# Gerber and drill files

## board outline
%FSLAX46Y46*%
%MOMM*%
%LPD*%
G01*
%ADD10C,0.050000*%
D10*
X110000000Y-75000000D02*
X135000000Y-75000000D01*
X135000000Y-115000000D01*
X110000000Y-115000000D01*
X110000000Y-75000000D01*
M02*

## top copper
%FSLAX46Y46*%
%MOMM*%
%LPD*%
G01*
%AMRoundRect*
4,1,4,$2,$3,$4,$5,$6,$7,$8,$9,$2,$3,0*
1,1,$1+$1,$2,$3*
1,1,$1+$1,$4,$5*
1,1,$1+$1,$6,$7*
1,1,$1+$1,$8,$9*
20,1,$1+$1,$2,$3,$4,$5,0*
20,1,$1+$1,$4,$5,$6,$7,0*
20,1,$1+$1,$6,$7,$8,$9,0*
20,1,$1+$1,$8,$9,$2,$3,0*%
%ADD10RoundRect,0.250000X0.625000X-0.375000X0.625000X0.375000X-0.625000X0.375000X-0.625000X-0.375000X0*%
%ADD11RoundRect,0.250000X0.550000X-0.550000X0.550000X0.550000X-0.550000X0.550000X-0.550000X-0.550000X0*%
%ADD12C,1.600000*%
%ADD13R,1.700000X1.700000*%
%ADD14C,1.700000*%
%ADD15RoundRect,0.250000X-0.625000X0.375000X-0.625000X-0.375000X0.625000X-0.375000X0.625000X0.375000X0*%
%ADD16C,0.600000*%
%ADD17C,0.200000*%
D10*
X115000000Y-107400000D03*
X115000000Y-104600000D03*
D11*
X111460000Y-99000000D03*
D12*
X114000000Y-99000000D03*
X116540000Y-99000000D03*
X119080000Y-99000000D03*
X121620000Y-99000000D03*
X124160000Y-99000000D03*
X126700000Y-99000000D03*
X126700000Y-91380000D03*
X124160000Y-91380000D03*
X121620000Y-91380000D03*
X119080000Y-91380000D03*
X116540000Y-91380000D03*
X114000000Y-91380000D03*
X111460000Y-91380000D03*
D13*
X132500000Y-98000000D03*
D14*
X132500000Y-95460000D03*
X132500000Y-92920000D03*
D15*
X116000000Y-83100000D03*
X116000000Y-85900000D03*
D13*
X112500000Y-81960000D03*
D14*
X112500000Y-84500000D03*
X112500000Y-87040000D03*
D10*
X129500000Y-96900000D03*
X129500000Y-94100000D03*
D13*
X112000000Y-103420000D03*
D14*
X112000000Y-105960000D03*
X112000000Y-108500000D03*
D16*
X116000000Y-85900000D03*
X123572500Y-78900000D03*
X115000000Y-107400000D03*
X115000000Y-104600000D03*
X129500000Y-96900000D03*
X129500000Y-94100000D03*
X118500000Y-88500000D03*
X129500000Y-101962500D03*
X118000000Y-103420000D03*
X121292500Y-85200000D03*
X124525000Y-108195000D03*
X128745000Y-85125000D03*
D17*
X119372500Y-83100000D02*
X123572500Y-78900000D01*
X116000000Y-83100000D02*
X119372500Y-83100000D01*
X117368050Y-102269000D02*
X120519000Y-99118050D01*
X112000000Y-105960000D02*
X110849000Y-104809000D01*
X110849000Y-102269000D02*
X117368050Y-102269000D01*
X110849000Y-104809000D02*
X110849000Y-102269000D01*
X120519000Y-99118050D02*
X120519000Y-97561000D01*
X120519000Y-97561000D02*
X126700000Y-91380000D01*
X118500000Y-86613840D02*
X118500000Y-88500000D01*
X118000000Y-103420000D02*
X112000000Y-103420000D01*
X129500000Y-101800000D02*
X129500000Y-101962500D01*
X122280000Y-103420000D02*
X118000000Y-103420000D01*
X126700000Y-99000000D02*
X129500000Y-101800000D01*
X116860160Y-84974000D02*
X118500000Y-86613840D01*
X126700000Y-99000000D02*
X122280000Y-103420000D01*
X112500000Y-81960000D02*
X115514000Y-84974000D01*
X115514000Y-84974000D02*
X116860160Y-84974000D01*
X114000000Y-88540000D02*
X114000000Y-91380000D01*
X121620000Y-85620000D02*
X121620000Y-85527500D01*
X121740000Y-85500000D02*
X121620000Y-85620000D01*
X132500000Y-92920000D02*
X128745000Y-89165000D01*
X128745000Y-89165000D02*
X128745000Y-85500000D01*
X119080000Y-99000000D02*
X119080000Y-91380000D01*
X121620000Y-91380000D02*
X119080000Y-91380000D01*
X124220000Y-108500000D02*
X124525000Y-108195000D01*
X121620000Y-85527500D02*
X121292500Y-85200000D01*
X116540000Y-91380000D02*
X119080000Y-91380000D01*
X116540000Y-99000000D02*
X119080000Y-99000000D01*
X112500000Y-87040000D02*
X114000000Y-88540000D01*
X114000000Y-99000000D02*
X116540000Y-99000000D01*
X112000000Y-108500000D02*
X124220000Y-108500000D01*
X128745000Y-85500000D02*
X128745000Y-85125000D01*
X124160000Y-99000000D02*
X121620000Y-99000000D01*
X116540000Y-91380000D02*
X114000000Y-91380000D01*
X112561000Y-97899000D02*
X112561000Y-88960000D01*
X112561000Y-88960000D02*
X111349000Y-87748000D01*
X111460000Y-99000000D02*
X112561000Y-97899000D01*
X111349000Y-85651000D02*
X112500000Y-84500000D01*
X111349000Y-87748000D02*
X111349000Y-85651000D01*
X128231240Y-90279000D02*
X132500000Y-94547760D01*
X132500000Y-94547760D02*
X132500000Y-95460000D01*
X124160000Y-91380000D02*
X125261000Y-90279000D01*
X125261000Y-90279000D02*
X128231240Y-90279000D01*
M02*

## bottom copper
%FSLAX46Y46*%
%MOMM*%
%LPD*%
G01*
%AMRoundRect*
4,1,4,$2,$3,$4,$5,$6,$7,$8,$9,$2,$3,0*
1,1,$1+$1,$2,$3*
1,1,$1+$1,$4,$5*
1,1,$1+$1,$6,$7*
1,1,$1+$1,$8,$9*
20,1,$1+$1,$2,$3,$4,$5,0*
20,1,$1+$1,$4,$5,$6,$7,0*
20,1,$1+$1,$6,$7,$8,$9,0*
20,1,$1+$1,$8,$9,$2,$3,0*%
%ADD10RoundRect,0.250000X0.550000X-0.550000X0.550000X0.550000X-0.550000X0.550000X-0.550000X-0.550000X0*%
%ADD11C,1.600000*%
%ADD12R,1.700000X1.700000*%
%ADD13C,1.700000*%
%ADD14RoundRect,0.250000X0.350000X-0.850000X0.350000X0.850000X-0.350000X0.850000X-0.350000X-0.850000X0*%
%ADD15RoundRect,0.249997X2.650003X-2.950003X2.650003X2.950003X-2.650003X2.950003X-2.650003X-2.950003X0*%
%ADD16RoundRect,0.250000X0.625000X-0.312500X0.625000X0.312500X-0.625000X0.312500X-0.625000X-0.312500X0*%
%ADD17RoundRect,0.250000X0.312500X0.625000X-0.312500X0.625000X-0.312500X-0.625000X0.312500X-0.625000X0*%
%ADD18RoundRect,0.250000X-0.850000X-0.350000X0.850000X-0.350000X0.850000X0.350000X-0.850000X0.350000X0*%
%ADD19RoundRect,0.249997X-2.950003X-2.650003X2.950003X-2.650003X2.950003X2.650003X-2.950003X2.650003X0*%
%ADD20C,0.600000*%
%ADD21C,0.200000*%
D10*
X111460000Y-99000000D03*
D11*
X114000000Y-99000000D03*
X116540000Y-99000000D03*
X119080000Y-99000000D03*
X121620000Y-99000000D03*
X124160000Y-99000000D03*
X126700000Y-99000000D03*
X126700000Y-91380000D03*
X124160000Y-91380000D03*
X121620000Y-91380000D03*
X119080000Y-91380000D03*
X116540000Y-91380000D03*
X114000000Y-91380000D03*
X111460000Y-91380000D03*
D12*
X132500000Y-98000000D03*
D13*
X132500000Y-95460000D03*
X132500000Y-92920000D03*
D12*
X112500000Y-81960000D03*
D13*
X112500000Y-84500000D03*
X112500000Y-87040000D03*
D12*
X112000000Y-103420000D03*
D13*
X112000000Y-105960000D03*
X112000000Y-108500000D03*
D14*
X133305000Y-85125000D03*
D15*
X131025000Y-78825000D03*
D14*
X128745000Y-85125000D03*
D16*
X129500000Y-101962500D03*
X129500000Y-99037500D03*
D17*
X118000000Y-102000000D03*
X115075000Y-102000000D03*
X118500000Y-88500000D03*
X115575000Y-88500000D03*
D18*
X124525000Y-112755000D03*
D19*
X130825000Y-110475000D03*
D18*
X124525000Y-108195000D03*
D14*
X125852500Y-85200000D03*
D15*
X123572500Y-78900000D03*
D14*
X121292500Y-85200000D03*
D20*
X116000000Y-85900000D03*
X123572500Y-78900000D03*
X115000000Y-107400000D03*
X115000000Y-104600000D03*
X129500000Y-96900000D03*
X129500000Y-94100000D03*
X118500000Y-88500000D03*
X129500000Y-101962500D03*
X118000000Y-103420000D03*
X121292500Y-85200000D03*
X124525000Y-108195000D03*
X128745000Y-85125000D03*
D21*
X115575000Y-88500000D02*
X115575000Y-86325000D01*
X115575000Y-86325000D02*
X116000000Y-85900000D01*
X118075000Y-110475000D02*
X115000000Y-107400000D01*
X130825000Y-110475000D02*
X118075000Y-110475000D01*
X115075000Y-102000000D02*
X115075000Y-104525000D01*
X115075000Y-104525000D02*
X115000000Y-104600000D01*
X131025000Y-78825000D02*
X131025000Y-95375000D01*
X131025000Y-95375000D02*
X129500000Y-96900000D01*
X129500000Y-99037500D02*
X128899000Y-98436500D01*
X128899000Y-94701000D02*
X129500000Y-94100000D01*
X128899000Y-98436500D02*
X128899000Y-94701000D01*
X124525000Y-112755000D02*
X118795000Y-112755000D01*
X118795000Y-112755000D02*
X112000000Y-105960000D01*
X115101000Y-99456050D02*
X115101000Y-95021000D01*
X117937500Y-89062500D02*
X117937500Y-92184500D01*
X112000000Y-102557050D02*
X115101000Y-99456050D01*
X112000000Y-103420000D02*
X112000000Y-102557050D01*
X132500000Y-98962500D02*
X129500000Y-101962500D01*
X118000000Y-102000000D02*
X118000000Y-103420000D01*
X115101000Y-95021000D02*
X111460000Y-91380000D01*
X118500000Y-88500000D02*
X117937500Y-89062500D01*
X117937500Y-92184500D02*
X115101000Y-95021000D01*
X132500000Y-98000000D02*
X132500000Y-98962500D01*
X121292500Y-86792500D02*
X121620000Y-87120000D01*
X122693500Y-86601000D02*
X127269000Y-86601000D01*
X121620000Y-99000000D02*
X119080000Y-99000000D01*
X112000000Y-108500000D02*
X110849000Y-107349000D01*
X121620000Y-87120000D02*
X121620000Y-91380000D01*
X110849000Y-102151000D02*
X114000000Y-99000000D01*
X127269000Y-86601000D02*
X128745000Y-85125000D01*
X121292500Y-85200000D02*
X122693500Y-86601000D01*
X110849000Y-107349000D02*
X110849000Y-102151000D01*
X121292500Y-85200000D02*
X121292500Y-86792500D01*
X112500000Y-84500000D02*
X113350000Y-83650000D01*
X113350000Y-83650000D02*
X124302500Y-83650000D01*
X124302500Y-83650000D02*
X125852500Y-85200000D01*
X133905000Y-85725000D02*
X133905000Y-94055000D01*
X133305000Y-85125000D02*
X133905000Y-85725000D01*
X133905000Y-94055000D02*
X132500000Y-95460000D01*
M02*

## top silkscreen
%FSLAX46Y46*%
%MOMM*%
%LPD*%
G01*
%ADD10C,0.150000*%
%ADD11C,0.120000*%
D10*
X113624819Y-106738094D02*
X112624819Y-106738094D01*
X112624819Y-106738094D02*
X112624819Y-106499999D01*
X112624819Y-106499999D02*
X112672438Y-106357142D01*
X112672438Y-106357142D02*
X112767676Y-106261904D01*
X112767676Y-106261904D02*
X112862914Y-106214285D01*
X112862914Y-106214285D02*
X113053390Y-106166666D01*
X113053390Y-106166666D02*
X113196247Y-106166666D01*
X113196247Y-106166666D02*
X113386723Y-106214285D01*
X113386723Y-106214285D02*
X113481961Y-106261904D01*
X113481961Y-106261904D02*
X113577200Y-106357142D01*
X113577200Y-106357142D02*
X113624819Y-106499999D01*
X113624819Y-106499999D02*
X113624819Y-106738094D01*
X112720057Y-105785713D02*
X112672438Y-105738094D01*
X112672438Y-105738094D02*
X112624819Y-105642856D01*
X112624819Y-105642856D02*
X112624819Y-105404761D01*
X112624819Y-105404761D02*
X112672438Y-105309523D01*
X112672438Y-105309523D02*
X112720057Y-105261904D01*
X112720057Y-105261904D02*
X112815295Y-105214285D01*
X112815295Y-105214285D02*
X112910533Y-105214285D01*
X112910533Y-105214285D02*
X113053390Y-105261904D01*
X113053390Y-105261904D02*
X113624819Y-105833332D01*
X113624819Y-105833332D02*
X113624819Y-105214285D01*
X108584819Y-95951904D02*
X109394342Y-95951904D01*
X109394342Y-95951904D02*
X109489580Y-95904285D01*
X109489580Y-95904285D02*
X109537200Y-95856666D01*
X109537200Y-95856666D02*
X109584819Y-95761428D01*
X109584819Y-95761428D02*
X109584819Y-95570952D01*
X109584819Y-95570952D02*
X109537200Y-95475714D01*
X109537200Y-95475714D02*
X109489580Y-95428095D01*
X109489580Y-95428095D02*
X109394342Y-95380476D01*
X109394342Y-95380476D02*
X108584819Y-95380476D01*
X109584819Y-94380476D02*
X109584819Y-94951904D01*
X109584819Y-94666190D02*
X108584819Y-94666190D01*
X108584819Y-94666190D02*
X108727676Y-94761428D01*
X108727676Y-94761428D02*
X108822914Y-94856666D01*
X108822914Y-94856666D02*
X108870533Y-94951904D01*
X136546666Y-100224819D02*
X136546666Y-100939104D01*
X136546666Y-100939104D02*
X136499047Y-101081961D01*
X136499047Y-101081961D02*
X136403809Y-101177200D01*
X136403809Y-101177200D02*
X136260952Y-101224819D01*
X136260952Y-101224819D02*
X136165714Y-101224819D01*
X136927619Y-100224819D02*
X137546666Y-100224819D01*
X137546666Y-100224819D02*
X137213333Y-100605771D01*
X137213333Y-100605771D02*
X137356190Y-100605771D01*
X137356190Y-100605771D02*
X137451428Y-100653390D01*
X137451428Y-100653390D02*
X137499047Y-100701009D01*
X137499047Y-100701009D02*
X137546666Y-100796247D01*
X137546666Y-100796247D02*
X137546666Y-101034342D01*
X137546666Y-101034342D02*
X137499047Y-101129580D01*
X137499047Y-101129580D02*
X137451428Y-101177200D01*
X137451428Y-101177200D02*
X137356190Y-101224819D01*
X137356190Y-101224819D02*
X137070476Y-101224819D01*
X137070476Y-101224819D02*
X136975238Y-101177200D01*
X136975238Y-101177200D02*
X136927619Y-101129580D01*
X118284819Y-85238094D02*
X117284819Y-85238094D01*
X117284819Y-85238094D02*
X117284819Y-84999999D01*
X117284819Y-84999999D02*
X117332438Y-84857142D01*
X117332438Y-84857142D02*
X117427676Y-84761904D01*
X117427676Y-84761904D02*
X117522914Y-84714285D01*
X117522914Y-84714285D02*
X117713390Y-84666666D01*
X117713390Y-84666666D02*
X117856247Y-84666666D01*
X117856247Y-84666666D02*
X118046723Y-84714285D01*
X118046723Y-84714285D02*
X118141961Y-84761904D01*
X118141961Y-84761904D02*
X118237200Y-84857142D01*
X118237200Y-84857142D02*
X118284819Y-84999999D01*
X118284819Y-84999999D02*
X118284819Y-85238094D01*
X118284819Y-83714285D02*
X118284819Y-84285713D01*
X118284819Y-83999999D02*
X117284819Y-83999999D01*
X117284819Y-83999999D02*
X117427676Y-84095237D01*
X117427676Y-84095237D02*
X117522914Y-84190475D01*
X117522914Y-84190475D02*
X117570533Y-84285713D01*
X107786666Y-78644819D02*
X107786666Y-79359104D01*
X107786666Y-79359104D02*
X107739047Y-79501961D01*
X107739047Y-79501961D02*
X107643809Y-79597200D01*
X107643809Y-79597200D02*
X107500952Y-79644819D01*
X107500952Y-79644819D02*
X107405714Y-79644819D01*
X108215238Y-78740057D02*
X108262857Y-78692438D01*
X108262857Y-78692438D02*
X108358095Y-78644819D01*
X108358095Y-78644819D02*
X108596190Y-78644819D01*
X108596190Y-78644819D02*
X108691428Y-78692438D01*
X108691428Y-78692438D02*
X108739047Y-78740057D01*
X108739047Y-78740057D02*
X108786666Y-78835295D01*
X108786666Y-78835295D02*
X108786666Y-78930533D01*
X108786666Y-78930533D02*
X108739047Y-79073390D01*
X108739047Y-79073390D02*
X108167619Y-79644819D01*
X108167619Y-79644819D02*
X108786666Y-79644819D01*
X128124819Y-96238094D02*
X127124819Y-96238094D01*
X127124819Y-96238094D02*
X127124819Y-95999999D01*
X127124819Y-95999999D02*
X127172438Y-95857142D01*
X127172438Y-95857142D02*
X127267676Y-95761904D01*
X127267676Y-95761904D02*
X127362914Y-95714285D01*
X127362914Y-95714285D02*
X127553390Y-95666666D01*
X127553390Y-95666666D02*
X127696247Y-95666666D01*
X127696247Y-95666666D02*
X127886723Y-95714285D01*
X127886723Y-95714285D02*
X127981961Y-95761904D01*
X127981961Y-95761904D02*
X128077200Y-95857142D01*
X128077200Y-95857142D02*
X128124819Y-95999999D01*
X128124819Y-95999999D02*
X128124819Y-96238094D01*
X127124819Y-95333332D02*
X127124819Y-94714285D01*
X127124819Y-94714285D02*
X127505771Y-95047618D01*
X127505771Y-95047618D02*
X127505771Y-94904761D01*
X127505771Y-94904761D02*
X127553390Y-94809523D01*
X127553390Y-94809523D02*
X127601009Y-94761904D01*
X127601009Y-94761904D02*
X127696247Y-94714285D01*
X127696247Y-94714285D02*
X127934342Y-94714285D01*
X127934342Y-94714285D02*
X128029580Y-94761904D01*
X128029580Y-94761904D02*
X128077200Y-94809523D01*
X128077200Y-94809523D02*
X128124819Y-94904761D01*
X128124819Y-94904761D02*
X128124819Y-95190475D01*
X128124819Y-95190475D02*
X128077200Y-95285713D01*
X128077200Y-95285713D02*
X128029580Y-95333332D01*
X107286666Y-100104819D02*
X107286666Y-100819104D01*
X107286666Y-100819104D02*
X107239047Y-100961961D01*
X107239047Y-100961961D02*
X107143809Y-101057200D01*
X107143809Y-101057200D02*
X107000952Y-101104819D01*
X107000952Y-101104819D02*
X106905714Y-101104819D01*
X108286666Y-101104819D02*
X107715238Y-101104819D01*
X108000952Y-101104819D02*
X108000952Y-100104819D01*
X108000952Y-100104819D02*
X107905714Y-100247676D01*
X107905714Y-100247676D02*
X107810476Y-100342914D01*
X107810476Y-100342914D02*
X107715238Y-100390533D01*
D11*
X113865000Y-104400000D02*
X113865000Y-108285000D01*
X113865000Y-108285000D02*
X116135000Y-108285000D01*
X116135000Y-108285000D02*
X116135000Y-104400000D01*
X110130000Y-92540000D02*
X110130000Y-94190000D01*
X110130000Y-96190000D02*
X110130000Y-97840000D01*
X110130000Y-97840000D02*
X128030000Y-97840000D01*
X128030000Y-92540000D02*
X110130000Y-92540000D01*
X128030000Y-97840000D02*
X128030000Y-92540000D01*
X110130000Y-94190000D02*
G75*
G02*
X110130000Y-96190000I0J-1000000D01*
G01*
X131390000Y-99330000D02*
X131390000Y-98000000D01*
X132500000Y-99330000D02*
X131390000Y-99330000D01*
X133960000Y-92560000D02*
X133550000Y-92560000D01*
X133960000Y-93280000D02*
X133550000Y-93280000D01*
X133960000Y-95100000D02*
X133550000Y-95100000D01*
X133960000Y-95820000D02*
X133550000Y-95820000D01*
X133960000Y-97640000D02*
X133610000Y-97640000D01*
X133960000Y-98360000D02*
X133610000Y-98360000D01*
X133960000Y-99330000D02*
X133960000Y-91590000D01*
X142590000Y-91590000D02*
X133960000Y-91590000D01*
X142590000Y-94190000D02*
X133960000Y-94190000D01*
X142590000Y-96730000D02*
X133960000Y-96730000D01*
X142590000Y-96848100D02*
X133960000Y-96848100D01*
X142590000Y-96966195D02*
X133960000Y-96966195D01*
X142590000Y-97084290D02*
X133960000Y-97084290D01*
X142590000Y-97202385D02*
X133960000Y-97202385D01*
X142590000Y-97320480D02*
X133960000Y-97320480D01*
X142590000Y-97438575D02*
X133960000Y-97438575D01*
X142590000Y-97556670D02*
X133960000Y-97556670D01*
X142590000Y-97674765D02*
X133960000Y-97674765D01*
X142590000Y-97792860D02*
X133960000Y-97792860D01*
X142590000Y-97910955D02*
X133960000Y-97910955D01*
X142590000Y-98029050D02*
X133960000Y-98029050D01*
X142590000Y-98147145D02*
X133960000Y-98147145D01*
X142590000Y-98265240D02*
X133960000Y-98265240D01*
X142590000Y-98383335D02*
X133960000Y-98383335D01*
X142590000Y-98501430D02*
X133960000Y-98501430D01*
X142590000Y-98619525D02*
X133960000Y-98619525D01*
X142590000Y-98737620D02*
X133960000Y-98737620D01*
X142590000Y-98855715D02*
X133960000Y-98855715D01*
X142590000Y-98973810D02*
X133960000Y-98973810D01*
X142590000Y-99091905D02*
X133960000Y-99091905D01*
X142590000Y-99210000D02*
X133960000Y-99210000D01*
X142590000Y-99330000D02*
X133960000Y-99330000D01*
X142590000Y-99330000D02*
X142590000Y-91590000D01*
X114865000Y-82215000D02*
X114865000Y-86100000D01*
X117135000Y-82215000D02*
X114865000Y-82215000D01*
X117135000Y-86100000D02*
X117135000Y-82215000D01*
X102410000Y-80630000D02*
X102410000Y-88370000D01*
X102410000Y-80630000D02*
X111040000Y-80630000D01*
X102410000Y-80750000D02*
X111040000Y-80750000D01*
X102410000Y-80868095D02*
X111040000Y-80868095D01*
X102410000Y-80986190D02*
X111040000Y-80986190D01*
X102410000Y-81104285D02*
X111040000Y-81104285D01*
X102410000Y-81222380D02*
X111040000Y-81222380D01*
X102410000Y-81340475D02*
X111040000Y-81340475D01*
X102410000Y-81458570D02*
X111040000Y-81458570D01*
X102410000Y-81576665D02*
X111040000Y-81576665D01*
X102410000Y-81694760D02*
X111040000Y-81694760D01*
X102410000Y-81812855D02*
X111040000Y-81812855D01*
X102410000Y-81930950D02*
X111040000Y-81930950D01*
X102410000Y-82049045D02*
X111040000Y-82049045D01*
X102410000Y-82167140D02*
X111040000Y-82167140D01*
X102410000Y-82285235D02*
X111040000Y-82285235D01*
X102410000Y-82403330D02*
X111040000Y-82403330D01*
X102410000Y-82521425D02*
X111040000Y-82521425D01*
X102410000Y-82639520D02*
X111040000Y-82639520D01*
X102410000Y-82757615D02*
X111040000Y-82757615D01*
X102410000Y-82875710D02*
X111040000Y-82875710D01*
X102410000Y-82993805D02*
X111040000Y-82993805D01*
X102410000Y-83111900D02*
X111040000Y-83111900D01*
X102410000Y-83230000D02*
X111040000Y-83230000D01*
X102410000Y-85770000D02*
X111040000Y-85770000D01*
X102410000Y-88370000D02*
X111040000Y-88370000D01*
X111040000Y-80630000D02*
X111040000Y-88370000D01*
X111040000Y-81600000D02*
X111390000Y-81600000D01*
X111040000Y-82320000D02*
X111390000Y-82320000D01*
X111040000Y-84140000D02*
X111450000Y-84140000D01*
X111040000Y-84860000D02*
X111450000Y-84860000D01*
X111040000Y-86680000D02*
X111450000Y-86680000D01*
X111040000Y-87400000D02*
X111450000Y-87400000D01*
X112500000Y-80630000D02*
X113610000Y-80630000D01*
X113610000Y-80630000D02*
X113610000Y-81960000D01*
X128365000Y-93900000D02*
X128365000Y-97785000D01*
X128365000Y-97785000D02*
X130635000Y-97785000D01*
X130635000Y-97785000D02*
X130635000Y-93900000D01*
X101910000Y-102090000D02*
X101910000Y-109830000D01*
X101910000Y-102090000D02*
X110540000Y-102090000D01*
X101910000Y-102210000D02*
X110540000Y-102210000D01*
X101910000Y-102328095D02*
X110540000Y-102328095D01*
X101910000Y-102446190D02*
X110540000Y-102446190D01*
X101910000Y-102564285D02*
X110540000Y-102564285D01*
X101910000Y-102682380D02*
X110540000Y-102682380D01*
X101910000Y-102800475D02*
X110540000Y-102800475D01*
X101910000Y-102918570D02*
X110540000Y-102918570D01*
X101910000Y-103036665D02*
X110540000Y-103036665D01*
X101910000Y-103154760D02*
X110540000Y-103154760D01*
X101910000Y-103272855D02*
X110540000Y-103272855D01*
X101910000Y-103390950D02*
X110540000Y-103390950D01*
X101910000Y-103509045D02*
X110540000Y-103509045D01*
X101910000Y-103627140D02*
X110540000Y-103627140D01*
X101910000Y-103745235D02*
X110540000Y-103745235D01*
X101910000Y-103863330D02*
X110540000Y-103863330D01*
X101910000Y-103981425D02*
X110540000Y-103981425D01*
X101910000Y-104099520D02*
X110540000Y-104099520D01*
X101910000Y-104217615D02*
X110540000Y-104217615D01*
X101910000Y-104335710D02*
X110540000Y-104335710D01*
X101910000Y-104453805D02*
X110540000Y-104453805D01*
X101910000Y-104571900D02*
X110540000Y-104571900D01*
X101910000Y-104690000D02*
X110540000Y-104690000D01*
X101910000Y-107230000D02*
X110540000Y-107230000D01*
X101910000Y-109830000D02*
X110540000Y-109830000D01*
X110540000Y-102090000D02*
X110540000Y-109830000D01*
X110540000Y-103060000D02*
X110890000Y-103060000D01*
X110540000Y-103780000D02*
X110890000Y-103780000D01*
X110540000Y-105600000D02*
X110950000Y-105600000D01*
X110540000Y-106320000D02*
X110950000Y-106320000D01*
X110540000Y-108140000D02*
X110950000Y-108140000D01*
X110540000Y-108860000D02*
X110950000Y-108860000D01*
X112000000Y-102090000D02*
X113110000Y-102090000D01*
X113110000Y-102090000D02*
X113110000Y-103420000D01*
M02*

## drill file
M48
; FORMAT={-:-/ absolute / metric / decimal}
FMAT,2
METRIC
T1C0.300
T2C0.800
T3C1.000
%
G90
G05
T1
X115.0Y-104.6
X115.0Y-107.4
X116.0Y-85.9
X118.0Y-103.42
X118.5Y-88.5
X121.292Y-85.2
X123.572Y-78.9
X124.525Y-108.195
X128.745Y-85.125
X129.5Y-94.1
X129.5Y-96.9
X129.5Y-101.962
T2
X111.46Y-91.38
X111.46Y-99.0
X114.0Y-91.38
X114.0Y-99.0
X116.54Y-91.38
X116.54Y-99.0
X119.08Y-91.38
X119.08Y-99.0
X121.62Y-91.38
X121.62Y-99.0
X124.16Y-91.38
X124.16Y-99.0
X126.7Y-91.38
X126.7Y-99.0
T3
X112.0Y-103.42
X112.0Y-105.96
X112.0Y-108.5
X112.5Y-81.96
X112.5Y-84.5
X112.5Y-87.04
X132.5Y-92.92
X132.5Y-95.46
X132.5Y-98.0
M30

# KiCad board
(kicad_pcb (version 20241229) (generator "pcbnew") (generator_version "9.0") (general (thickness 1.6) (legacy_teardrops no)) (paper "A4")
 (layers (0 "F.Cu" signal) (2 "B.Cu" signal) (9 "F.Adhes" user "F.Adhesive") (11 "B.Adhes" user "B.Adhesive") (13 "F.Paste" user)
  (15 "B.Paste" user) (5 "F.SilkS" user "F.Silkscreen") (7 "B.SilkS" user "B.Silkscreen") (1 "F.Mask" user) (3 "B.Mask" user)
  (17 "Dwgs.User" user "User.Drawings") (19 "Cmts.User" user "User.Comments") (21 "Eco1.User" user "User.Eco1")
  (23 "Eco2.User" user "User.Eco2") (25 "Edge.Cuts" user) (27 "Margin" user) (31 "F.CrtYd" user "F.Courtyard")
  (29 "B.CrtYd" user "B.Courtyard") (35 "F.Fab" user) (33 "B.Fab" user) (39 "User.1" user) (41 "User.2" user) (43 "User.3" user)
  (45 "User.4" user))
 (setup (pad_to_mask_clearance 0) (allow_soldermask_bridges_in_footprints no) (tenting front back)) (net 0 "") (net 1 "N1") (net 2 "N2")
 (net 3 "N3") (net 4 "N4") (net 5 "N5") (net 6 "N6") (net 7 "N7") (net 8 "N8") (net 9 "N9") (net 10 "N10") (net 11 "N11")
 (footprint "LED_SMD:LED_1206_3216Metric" (layer "F.Cu") (at 115 106 90)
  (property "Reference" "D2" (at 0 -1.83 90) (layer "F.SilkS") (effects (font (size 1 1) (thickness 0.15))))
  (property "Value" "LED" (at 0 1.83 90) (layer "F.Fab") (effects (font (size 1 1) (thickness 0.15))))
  (fp_line (start 1.6 -1.135) (end -2.285 -1.135) (stroke (width 0.12) (type solid)) (layer "F.SilkS"))
  (fp_line (start -2.285 -1.135) (end -2.285 1.135) (stroke (width 0.12) (type solid)) (layer "F.SilkS"))
  (fp_line (start -2.285 1.135) (end 1.6 1.135) (stroke (width 0.12) (type solid)) (layer "F.SilkS"))
  (pad "1" smd roundrect (at -1.4 0 90) (size 1.25 1.75) (layers "F.Cu" "F.Mask" "F.Paste") (roundrect_rratio 0.2) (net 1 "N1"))
  (pad "2" smd roundrect (at 1.4 0 90) (size 1.25 1.75) (layers "F.Cu" "F.Mask" "F.Paste") (roundrect_rratio 0.2) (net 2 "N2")))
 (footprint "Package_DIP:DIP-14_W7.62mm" (layer "F.Cu") (at 111.46 99 90)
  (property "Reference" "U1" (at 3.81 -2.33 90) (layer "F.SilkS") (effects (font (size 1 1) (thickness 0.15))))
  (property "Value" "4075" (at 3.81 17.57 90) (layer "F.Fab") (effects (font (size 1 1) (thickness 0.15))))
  (fp_line (start 6.46 -1.33) (end 4.81 -1.33) (stroke (width 0.12) (type solid)) (layer "F.SilkS"))
  (fp_line (start 2.81 -1.33) (end 1.16 -1.33) (stroke (width 0.12) (type solid)) (layer "F.SilkS"))
  (fp_line (start 1.16 -1.33) (end 1.16 16.57) (stroke (width 0.12) (type solid)) (layer "F.SilkS"))
  (fp_line (start 6.46 16.57) (end 6.46 -1.33) (stroke (width 0.12) (type solid)) (layer "F.SilkS"))
  (fp_line (start 1.16 16.57) (end 6.46 16.57) (stroke (width 0.12) (type solid)) (layer "F.SilkS"))
  (fp_arc (start 4.81 -1.33) (mid 3.81 -0.33) (end 2.81 -1.33) (stroke (width 0.12) (type solid)) (layer "F.SilkS"))
  (pad "1" thru_hole roundrect (at 0 0 90) (size 1.6 1.6) (drill 0.8) (layers "*.Cu" "*.Mask") (remove_unused_layers no)
   (roundrect_rratio 0.15625) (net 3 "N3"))
  (pad "2" thru_hole circle (at 0 2.54 90) (size 1.6 1.6) (drill 0.8) (layers "*.Cu" "*.Mask") (remove_unused_layers no) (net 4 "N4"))
  (pad "3" thru_hole circle (at 0 5.08 90) (size 1.6 1.6) (drill 0.8) (layers "*.Cu" "*.Mask") (remove_unused_layers no) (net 4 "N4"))
  (pad "4" thru_hole circle (at 0 7.62 90) (size 1.6 1.6) (drill 0.8) (layers "*.Cu" "*.Mask") (remove_unused_layers no) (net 4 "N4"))
  (pad "5" thru_hole circle (at 0 10.16 90) (size 1.6 1.6) (drill 0.8) (layers "*.Cu" "*.Mask") (remove_unused_layers no) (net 4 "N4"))
  (pad "6" thru_hole circle (at 0 12.7 90) (size 1.6 1.6) (drill 0.8) (layers "*.Cu" "*.Mask") (remove_unused_layers no) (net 4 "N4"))
  (pad "7" thru_hole circle (at 0 15.24 90) (size 1.6 1.6) (drill 0.8) (layers "*.Cu" "*.Mask") (remove_unused_layers no) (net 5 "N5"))
  (pad "8" thru_hole circle (at 7.62 15.24 90) (size 1.6 1.6) (drill 0.8) (layers "*.Cu" "*.Mask") (remove_unused_layers no) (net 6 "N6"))
  (pad "9" thru_hole circle (at 7.62 12.7 90) (size 1.6 1.6) (drill 0.8) (layers "*.Cu" "*.Mask") (remove_unused_layers no) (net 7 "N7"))
  (pad "10" thru_hole circle (at 7.62 10.16 90) (size 1.6 1.6) (drill 0.8) (layers "*.Cu" "*.Mask") (remove_unused_layers no) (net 4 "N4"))
  (pad "11" thru_hole circle (at 7.62 7.62 90) (size 1.6 1.6) (drill 0.8) (layers "*.Cu" "*.Mask") (remove_unused_layers no) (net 4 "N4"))
  (pad "12" thru_hole circle (at 7.62 5.08 90) (size 1.6 1.6) (drill 0.8) (layers "*.Cu" "*.Mask") (remove_unused_layers no) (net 4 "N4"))
  (pad "13" thru_hole circle (at 7.62 2.54 90) (size 1.6 1.6) (drill 0.8) (layers "*.Cu" "*.Mask") (remove_unused_layers no) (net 4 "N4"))
  (pad "14" thru_hole circle (at 7.62 0 90) (size 1.6 1.6) (drill 0.8) (layers "*.Cu" "*.Mask") (remove_unused_layers no) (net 5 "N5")))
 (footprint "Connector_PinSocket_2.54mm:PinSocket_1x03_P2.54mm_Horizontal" (layer "F.Cu") (at 132.5 98 180)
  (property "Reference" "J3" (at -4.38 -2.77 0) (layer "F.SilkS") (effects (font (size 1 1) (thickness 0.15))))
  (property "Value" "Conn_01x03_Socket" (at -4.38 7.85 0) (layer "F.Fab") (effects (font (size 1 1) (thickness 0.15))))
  (fp_line (start 1.11 -1.33) (end 1.11 0) (stroke (width 0.12) (type solid)) (layer "F.SilkS"))
  (fp_line (start 0 -1.33) (end 1.11 -1.33) (stroke (width 0.12) (type solid)) (layer "F.SilkS"))
  (fp_line (start -1.46 5.44) (end -1.05 5.44) (stroke (width 0.12) (type solid)) (layer "F.SilkS"))
  (fp_line (start -1.46 4.72) (end -1.05 4.72) (stroke (width 0.12) (type solid)) (layer "F.SilkS"))
  (fp_line (start -1.46 2.9) (end -1.05 2.9) (stroke (width 0.12) (type solid)) (layer "F.SilkS"))
  (fp_line (start -1.46 2.18) (end -1.05 2.18) (stroke (width 0.12) (type solid)) (layer "F.SilkS"))
  (fp_line (start -1.46 0.36) (end -1.11 0.36) (stroke (width 0.12) (type solid)) (layer "F.SilkS"))
  (fp_line (start -1.46 -0.36) (end -1.11 -0.36) (stroke (width 0.12) (type solid)) (layer "F.SilkS"))
  (fp_line (start -1.46 -1.33) (end -1.46 6.41) (stroke (width 0.12) (type solid)) (layer "F.SilkS"))
  (fp_line (start -10.09 6.41) (end -1.46 6.41) (stroke (width 0.12) (type solid)) (layer "F.SilkS"))
  (fp_line (start -10.09 3.81) (end -1.46 3.81) (stroke (width 0.12) (type solid)) (layer "F.SilkS"))
  (fp_line (start -10.09 1.27) (end -1.46 1.27) (stroke (width 0.12) (type solid)) (layer "F.SilkS"))
  (fp_line (start -10.09 1.1519) (end -1.46 1.1519) (stroke (width 0.12) (type solid)) (layer "F.SilkS"))
  (fp_line (start -10.09 1.033805) (end -1.46 1.033805) (stroke (width 0.12) (type solid)) (layer "F.SilkS"))
  (fp_line (start -10.09 0.91571) (end -1.46 0.91571) (stroke (width 0.12) (type solid)) (layer "F.SilkS"))
  (fp_line (start -10.09 0.797615) (end -1.46 0.797615) (stroke (width 0.12) (type solid)) (layer "F.SilkS"))
  (fp_line (start -10.09 0.67952) (end -1.46 0.67952) (stroke (width 0.12) (type solid)) (layer "F.SilkS"))
  (fp_line (start -10.09 0.561425) (end -1.46 0.561425) (stroke (width 0.12) (type solid)) (layer "F.SilkS"))
  (fp_line (start -10.09 0.44333) (end -1.46 0.44333) (stroke (width 0.12) (type solid)) (layer "F.SilkS"))
  (fp_line (start -10.09 0.325235) (end -1.46 0.325235) (stroke (width 0.12) (type solid)) (layer "F.SilkS"))
  (fp_line (start -10.09 0.20714) (end -1.46 0.20714) (stroke (width 0.12) (type solid)) (layer "F.SilkS"))
  (fp_line (start -10.09 0.089045) (end -1.46 0.089045) (stroke (width 0.12) (type solid)) (layer "F.SilkS"))
  (fp_line (start -10.09 -0.02905) (end -1.46 -0.02905) (stroke (width 0.12) (type solid)) (layer "F.SilkS"))
  (fp_line (start -10.09 -0.147145) (end -1.46 -0.147145) (stroke (width 0.12) (type solid)) (layer "F.SilkS"))
  (fp_line (start -10.09 -0.26524) (end -1.46 -0.26524) (stroke (width 0.12) (type solid)) (layer "F.SilkS"))
  (fp_line (start -10.09 -0.383335) (end -1.46 -0.383335) (stroke (width 0.12) (type solid)) (layer "F.SilkS"))
  (fp_line (start -10.09 -0.50143) (end -1.46 -0.50143) (stroke (width 0.12) (type solid)) (layer "F.SilkS"))
  (fp_line (start -10.09 -0.619525) (end -1.46 -0.619525) (stroke (width 0.12) (type solid)) (layer "F.SilkS"))
  (fp_line (start -10.09 -0.73762) (end -1.46 -0.73762) (stroke (width 0.12) (type solid)) (layer "F.SilkS"))
  (fp_line (start -10.09 -0.855715) (end -1.46 -0.855715) (stroke (width 0.12) (type solid)) (layer "F.SilkS"))
  (fp_line (start -10.09 -0.97381) (end -1.46 -0.97381) (stroke (width 0.12) (type solid)) (layer "F.SilkS"))
  (fp_line (start -10.09 -1.091905) (end -1.46 -1.091905) (stroke (width 0.12) (type solid)) (layer "F.SilkS"))
  (fp_line (start -10.09 -1.21) (end -1.46 -1.21) (stroke (width 0.12) (type solid)) (layer "F.SilkS"))
  (fp_line (start -10.09 -1.33) (end -1.46 -1.33) (stroke (width 0.12) (type solid)) (layer "F.SilkS"))
  (fp_line (start -10.09 -1.33) (end -10.09 6.41) (stroke (width 0.12) (type solid)) (layer "F.SilkS"))
  (pad "1" thru_hole rect (at 0 0 180) (size 1.7 1.7) (drill 1) (layers "*.Cu" "*.Mask") (remove_unused_layers no) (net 5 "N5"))
  (pad "2" thru_hole circle (at 0 2.54 180) (size 1.7 1.7) (drill 1) (layers "*.Cu" "*.Mask") (remove_unused_layers no) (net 7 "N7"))
  (pad "3" thru_hole circle (at 0 5.08 180) (size 1.7 1.7) (drill 1) (layers "*.Cu" "*.Mask") (remove_unused_layers no) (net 4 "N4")))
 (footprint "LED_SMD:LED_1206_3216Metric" (layer "F.Cu") (at 116 84.5 -90)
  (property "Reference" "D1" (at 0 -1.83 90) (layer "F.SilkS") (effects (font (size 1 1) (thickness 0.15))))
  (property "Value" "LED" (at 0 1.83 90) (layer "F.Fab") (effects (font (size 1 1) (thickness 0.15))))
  (fp_line (start -2.285 1.135) (end 1.6 1.135) (stroke (width 0.12) (type solid)) (layer "F.SilkS"))
  (fp_line (start -2.285 -1.135) (end -2.285 1.135) (stroke (width 0.12) (type solid)) (layer "F.SilkS"))
  (fp_line (start 1.6 -1.135) (end -2.285 -1.135) (stroke (width 0.12) (type solid)) (layer "F.SilkS"))
  (pad "1" smd roundrect (at -1.4 0 270) (size 1.25 1.75) (layers "F.Cu" "F.Mask" "F.Paste") (roundrect_rratio 0.2) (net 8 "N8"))
  (pad "2" smd roundrect (at 1.4 0 270) (size 1.25 1.75) (layers "F.Cu" "F.Mask" "F.Paste") (roundrect_rratio 0.2) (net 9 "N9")))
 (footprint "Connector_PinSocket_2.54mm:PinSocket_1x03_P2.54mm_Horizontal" (layer "F.Cu") (at 112.5 81.96)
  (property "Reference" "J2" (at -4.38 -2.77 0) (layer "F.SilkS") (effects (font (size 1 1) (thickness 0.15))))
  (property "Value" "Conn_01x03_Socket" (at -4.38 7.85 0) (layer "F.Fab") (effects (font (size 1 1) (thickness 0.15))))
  (fp_line (start -10.09 -1.33) (end -10.09 6.41) (stroke (width 0.12) (type solid)) (layer "F.SilkS"))
  (fp_line (start -10.09 -1.33) (end -1.46 -1.33) (stroke (width 0.12) (type solid)) (layer "F.SilkS"))
  (fp_line (start -10.09 -1.21) (end -1.46 -1.21) (stroke (width 0.12) (type solid)) (layer "F.SilkS"))
  (fp_line (start -10.09 -1.091905) (end -1.46 -1.091905) (stroke (width 0.12) (type solid)) (layer "F.SilkS"))
  (fp_line (start -10.09 -0.97381) (end -1.46 -0.97381) (stroke (width 0.12) (type solid)) (layer "F.SilkS"))
  (fp_line (start -10.09 -0.855715) (end -1.46 -0.855715) (stroke (width 0.12) (type solid)) (layer "F.SilkS"))
  (fp_line (start -10.09 -0.73762) (end -1.46 -0.73762) (stroke (width 0.12) (type solid)) (layer "F.SilkS"))
  (fp_line (start -10.09 -0.619525) (end -1.46 -0.619525) (stroke (width 0.12) (type solid)) (layer "F.SilkS"))
  (fp_line (start -10.09 -0.50143) (end -1.46 -0.50143) (stroke (width 0.12) (type solid)) (layer "F.SilkS"))
  (fp_line (start -10.09 -0.383335) (end -1.46 -0.383335) (stroke (width 0.12) (type solid)) (layer "F.SilkS"))
  (fp_line (start -10.09 -0.26524) (end -1.46 -0.26524) (stroke (width 0.12) (type solid)) (layer "F.SilkS"))
  (fp_line (start -10.09 -0.147145) (end -1.46 -0.147145) (stroke (width 0.12) (type solid)) (layer "F.SilkS"))
  (fp_line (start -10.09 -0.02905) (end -1.46 -0.02905) (stroke (width 0.12) (type solid)) (layer "F.SilkS"))
  (fp_line (start -10.09 0.089045) (end -1.46 0.089045) (stroke (width 0.12) (type solid)) (layer "F.SilkS"))
  (fp_line (start -10.09 0.20714) (end -1.46 0.20714) (stroke (width 0.12) (type solid)) (layer "F.SilkS"))
  (fp_line (start -10.09 0.325235) (end -1.46 0.325235) (stroke (width 0.12) (type solid)) (layer "F.SilkS"))
  (fp_line (start -10.09 0.44333) (end -1.46 0.44333) (stroke (width 0.12) (type solid)) (layer "F.SilkS"))
  (fp_line (start -10.09 0.561425) (end -1.46 0.561425) (stroke (width 0.12) (type solid)) (layer "F.SilkS"))
  (fp_line (start -10.09 0.67952) (end -1.46 0.67952) (stroke (width 0.12) (type solid)) (layer "F.SilkS"))
  (fp_line (start -10.09 0.797615) (end -1.46 0.797615) (stroke (width 0.12) (type solid)) (layer "F.SilkS"))
  (fp_line (start -10.09 0.91571) (end -1.46 0.91571) (stroke (width 0.12) (type solid)) (layer "F.SilkS"))
  (fp_line (start -10.09 1.033805) (end -1.46 1.033805) (stroke (width 0.12) (type solid)) (layer "F.SilkS"))
  (fp_line (start -10.09 1.1519) (end -1.46 1.1519) (stroke (width 0.12) (type solid)) (layer "F.SilkS"))
  (fp_line (start -10.09 1.27) (end -1.46 1.27) (stroke (width 0.12) (type solid)) (layer "F.SilkS"))
  (fp_line (start -10.09 3.81) (end -1.46 3.81) (stroke (width 0.12) (type solid)) (layer "F.SilkS"))
  (fp_line (start -10.09 6.41) (end -1.46 6.41) (stroke (width 0.12) (type solid)) (layer "F.SilkS"))
  (fp_line (start -1.46 -1.33) (end -1.46 6.41) (stroke (width 0.12) (type solid)) (layer "F.SilkS"))
  (fp_line (start -1.46 -0.36) (end -1.11 -0.36) (stroke (width 0.12) (type solid)) (layer "F.SilkS"))
  (fp_line (start -1.46 0.36) (end -1.11 0.36) (stroke (width 0.12) (type solid)) (layer "F.SilkS"))
  (fp_line (start -1.46 2.18) (end -1.05 2.18) (stroke (width 0.12) (type solid)) (layer "F.SilkS"))
  (fp_line (start -1.46 2.9) (end -1.05 2.9) (stroke (width 0.12) (type solid)) (layer "F.SilkS"))
  (fp_line (start -1.46 4.72) (end -1.05 4.72) (stroke (width 0.12) (type solid)) (layer "F.SilkS"))
  (fp_line (start -1.46 5.44) (end -1.05 5.44) (stroke (width 0.12) (type solid)) (layer "F.SilkS"))
  (fp_line (start 0 -1.33) (end 1.11 -1.33) (stroke (width 0.12) (type solid)) (layer "F.SilkS"))
  (fp_line (start 1.11 -1.33) (end 1.11 0) (stroke (width 0.12) (type solid)) (layer "F.SilkS"))
  (pad "1" thru_hole rect (at 0 0) (size 1.7 1.7) (drill 1) (layers "*.Cu" "*.Mask") (remove_unused_layers no) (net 5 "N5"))
  (pad "2" thru_hole circle (at 0 2.54) (size 1.7 1.7) (drill 1) (layers "*.Cu" "*.Mask") (remove_unused_layers no) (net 3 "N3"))
  (pad "3" thru_hole circle (at 0 5.08) (size 1.7 1.7) (drill 1) (layers "*.Cu" "*.Mask") (remove_unused_layers no) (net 4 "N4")))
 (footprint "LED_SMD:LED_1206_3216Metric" (layer "F.Cu") (at 129.5 95.5 90)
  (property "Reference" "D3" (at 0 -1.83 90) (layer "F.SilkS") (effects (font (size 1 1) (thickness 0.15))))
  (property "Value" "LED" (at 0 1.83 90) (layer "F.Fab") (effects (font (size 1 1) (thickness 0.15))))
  (fp_line (start 1.6 -1.135) (end -2.285 -1.135) (stroke (width 0.12) (type solid)) (layer "F.SilkS"))
  (fp_line (start -2.285 -1.135) (end -2.285 1.135) (stroke (width 0.12) (type solid)) (layer "F.SilkS"))
  (fp_line (start -2.285 1.135) (end 1.6 1.135) (stroke (width 0.12) (type solid)) (layer "F.SilkS"))
  (pad "1" smd roundrect (at -1.4 0 90) (size 1.25 1.75) (layers "F.Cu" "F.Mask" "F.Paste") (roundrect_rratio 0.2) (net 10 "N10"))
  (pad "2" smd roundrect (at 1.4 0 90) (size 1.25 1.75) (layers "F.Cu" "F.Mask" "F.Paste") (roundrect_rratio 0.2) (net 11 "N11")))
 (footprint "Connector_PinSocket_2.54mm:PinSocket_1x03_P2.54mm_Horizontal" (layer "F.Cu") (at 112 103.42)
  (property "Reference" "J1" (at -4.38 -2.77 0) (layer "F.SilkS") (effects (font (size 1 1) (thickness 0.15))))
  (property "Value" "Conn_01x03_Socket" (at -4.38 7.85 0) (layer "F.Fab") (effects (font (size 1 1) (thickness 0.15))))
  (fp_line (start -10.09 -1.33) (end -10.09 6.41) (stroke (width 0.12) (type solid)) (layer "F.SilkS"))
  (fp_line (start -10.09 -1.33) (end -1.46 -1.33) (stroke (width 0.12) (type solid)) (layer "F.SilkS"))
  (fp_line (start -10.09 -1.21) (end -1.46 -1.21) (stroke (width 0.12) (type solid)) (layer "F.SilkS"))
  (fp_line (start -10.09 -1.091905) (end -1.46 -1.091905) (stroke (width 0.12) (type solid)) (layer "F.SilkS"))
  (fp_line (start -10.09 -0.97381) (end -1.46 -0.97381) (stroke (width 0.12) (type solid)) (layer "F.SilkS"))
  (fp_line (start -10.09 -0.855715) (end -1.46 -0.855715) (stroke (width 0.12) (type solid)) (layer "F.SilkS"))
  (fp_line (start -10.09 -0.73762) (end -1.46 -0.73762) (stroke (width 0.12) (type solid)) (layer "F.SilkS"))
  (fp_line (start -10.09 -0.619525) (end -1.46 -0.619525) (stroke (width 0.12) (type solid)) (layer "F.SilkS"))
  (fp_line (start -10.09 -0.50143) (end -1.46 -0.50143) (stroke (width 0.12) (type solid)) (layer "F.SilkS"))
  (fp_line (start -10.09 -0.383335) (end -1.46 -0.383335) (stroke (width 0.12) (type solid)) (layer "F.SilkS"))
  (fp_line (start -10.09 -0.26524) (end -1.46 -0.26524) (stroke (width 0.12) (type solid)) (layer "F.SilkS"))
  (fp_line (start -10.09 -0.147145) (end -1.46 -0.147145) (stroke (width 0.12) (type solid)) (layer "F.SilkS"))
  (fp_line (start -10.09 -0.02905) (end -1.46 -0.02905) (stroke (width 0.12) (type solid)) (layer "F.SilkS"))
  (fp_line (start -10.09 0.089045) (end -1.46 0.089045) (stroke (width 0.12) (type solid)) (layer "F.SilkS"))
  (fp_line (start -10.09 0.20714) (end -1.46 0.20714) (stroke (width 0.12) (type solid)) (layer "F.SilkS"))
  (fp_line (start -10.09 0.325235) (end -1.46 0.325235) (stroke (width 0.12) (type solid)) (layer "F.SilkS"))
  (fp_line (start -10.09 0.44333) (end -1.46 0.44333) (stroke (width 0.12) (type solid)) (layer "F.SilkS"))
  (fp_line (start -10.09 0.561425) (end -1.46 0.561425) (stroke (width 0.12) (type solid)) (layer "F.SilkS"))
  (fp_line (start -10.09 0.67952) (end -1.46 0.67952) (stroke (width 0.12) (type solid)) (layer "F.SilkS"))
  (fp_line (start -10.09 0.797615) (end -1.46 0.797615) (stroke (width 0.12) (type solid)) (layer "F.SilkS"))
  (fp_line (start -10.09 0.91571) (end -1.46 0.91571) (stroke (width 0.12) (type solid)) (layer "F.SilkS"))
  (fp_line (start -10.09 1.033805) (end -1.46 1.033805) (stroke (width 0.12) (type solid)) (layer "F.SilkS"))
  (fp_line (start -10.09 1.1519) (end -1.46 1.1519) (stroke (width 0.12) (type solid)) (layer "F.SilkS"))
  (fp_line (start -10.09 1.27) (end -1.46 1.27) (stroke (width 0.12) (type solid)) (layer "F.SilkS"))
  (fp_line (start -10.09 3.81) (end -1.46 3.81) (stroke (width 0.12) (type solid)) (layer "F.SilkS"))
  (fp_line (start -10.09 6.41) (end -1.46 6.41) (stroke (width 0.12) (type solid)) (layer "F.SilkS"))
  (fp_line (start -1.46 -1.33) (end -1.46 6.41) (stroke (width 0.12) (type solid)) (layer "F.SilkS"))
  (fp_line (start -1.46 -0.36) (end -1.11 -0.36) (stroke (width 0.12) (type solid)) (layer "F.SilkS"))
  (fp_line (start -1.46 0.36) (end -1.11 0.36) (stroke (width 0.12) (type solid)) (layer "F.SilkS"))
  (fp_line (start -1.46 2.18) (end -1.05 2.18) (stroke (width 0.12) (type solid)) (layer "F.SilkS"))
  (fp_line (start -1.46 2.9) (end -1.05 2.9) (stroke (width 0.12) (type solid)) (layer "F.SilkS"))
  (fp_line (start -1.46 4.72) (end -1.05 4.72) (stroke (width 0.12) (type solid)) (layer "F.SilkS"))
  (fp_line (start -1.46 5.44) (end -1.05 5.44) (stroke (width 0.12) (type solid)) (layer "F.SilkS"))
  (fp_line (start 0 -1.33) (end 1.11 -1.33) (stroke (width 0.12) (type solid)) (layer "F.SilkS"))
  (fp_line (start 1.11 -1.33) (end 1.11 0) (stroke (width 0.12) (type solid)) (layer "F.SilkS"))
  (pad "1" thru_hole rect (at 0 0) (size 1.7 1.7) (drill 1) (layers "*.Cu" "*.Mask") (remove_unused_layers no) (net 5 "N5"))
  (pad "2" thru_hole circle (at 0 2.54) (size 1.7 1.7) (drill 1) (layers "*.Cu" "*.Mask") (remove_unused_layers no) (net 6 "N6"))
  (pad "3" thru_hole circle (at 0 5.08) (size 1.7 1.7) (drill 1) (layers "*.Cu" "*.Mask") (remove_unused_layers no) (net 4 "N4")))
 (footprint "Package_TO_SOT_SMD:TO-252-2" (layer "B.Cu") (at 131.025 80.085 90)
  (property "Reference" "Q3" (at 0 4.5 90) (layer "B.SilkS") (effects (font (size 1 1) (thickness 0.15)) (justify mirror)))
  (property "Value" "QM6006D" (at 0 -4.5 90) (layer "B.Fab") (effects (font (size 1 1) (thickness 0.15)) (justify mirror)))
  (pad "" smd roundrect (at -0.415 -1.525 90) (size 3.05 2.75) (layers "B.Paste") (roundrect_rratio 0.090909))
  (pad "" smd roundrect (at -0.415 1.525 90) (size 3.05 2.75) (layers "B.Paste") (roundrect_rratio 0.090909))
  (pad "" smd roundrect (at 2.935 -1.525 90) (size 3.05 2.75) (layers "B.Paste") (roundrect_rratio 0.090909))
  (pad "" smd roundrect (at 2.935 1.525 90) (size 3.05 2.75) (layers "B.Paste") (roundrect_rratio 0.090909))
  (pad "1" smd roundrect (at -5.04 2.28 90) (size 2.2 1.2) (layers "B.Cu" "B.Mask" "B.Paste") (roundrect_rratio 0.208333) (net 7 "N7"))
  (pad "2" smd roundrect (at 1.26 0 90) (size 6.4 5.8) (layers "B.Cu" "B.Mask") (roundrect_rratio 0.043103) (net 10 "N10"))
  (pad "3" smd roundrect (at -5.04 -2.28 90) (size 2.2 1.2) (layers "B.Cu" "B.Mask" "B.Paste") (roundrect_rratio 0.208333) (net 4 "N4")))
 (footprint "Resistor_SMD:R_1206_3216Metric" (layer "B.Cu") (at 129.5 100.5 90)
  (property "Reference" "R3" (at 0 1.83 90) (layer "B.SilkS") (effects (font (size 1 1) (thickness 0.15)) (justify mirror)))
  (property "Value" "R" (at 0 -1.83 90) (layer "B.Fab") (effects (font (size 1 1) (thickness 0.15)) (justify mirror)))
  (pad "1" smd roundrect (at -1.4625 0 90) (size 1.125 1.75) (layers "B.Cu" "B.Mask" "B.Paste") (roundrect_rratio 0.222222) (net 5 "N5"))
  (pad "2" smd roundrect (at 1.4625 0 90) (size 1.125 1.75) (layers "B.Cu" "B.Mask" "B.Paste") (roundrect_rratio 0.222222) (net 11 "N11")))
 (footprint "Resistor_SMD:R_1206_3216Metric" (layer "B.Cu") (at 116.5375 102 180)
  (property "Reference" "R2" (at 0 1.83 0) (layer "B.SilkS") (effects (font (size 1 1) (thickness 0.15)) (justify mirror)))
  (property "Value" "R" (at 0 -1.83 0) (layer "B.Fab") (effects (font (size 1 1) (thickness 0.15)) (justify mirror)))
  (pad "1" smd roundrect (at -1.4625 0 180) (size 1.125 1.75) (layers "B.Cu" "B.Mask" "B.Paste") (roundrect_rratio 0.222222) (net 5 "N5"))
  (pad "2" smd roundrect (at 1.4625 0 180) (size 1.125 1.75) (layers "B.Cu" "B.Mask" "B.Paste") (roundrect_rratio 0.222222) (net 2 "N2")))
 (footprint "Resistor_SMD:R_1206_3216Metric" (layer "B.Cu") (at 117.0375 88.5 180)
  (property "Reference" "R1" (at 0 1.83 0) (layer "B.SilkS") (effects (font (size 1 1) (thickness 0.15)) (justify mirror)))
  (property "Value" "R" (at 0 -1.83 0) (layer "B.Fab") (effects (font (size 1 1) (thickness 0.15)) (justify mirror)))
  (pad "1" smd roundrect (at -1.4625 0 180) (size 1.125 1.75) (layers "B.Cu" "B.Mask" "B.Paste") (roundrect_rratio 0.222222) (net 5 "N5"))
  (pad "2" smd roundrect (at 1.4625 0 180) (size 1.125 1.75) (layers "B.Cu" "B.Mask" "B.Paste") (roundrect_rratio 0.222222) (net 9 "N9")))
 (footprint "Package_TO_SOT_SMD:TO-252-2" (layer "B.Cu") (at 129.565 110.475)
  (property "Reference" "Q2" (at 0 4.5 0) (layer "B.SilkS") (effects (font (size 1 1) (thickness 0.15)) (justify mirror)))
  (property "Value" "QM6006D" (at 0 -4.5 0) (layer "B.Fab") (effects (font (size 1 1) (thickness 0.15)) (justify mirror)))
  (pad "" smd roundrect (at -0.415 -1.525) (size 3.05 2.75) (layers "B.Paste") (roundrect_rratio 0.090909))
  (pad "" smd roundrect (at -0.415 1.525) (size 3.05 2.75) (layers "B.Paste") (roundrect_rratio 0.090909))
  (pad "" smd roundrect (at 2.935 -1.525) (size 3.05 2.75) (layers "B.Paste") (roundrect_rratio 0.090909))
  (pad "" smd roundrect (at 2.935 1.525) (size 3.05 2.75) (layers "B.Paste") (roundrect_rratio 0.090909))
  (pad "1" smd roundrect (at -5.04 2.28) (size 2.2 1.2) (layers "B.Cu" "B.Mask" "B.Paste") (roundrect_rratio 0.208333) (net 6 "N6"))
  (pad "2" smd roundrect (at 1.26 0) (size 6.4 5.8) (layers "B.Cu" "B.Mask") (roundrect_rratio 0.043103) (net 1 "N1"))
  (pad "3" smd roundrect (at -5.04 -2.28) (size 2.2 1.2) (layers "B.Cu" "B.Mask" "B.Paste") (roundrect_rratio 0.208333) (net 4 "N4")))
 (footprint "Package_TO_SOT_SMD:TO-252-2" (layer "B.Cu") (at 123.5725 80.16 90)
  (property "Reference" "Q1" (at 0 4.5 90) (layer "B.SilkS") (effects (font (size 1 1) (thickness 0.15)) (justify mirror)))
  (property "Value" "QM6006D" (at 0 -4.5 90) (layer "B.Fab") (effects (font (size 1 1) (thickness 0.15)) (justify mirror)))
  (pad "" smd roundrect (at -0.415 -1.525 90) (size 3.05 2.75) (layers "B.Paste") (roundrect_rratio 0.090909))
  (pad "" smd roundrect (at -0.415 1.525 90) (size 3.05 2.75) (layers "B.Paste") (roundrect_rratio 0.090909))
  (pad "" smd roundrect (at 2.935 -1.525 90) (size 3.05 2.75) (layers "B.Paste") (roundrect_rratio 0.090909))
  (pad "" smd roundrect (at 2.935 1.525 90) (size 3.05 2.75) (layers "B.Paste") (roundrect_rratio 0.090909))
  (pad "1" smd roundrect (at -5.04 2.28 90) (size 2.2 1.2) (layers "B.Cu" "B.Mask" "B.Paste") (roundrect_rratio 0.208333) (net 3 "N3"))
  (pad "2" smd roundrect (at 1.26 0 90) (size 6.4 5.8) (layers "B.Cu" "B.Mask") (roundrect_rratio 0.043103) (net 8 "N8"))
  (pad "3" smd roundrect (at -5.04 -2.28 90) (size 2.2 1.2) (layers "B.Cu" "B.Mask" "B.Paste") (roundrect_rratio 0.208333) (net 4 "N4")))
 (gr_rect (start 110 75) (end 135 115) (stroke (width 0.05) (type default)) (fill no) (layer "Edge.Cuts"))
 (via (at 116 85.9) (size 0.6) (drill 0.3) (layers "F.Cu" "B.Cu") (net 9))
 (segment (start 115.575 88.5) (end 115.575 86.325) (width 0.2) (layer "B.Cu") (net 9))
 (segment (start 115.575 86.325) (end 116 85.9) (width 0.2) (layer "B.Cu") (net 9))
 (segment (start 119.3725 83.1) (end 123.5725 78.9) (width 0.2) (layer "F.Cu") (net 8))
 (segment (start 116 83.1) (end 119.3725 83.1) (width 0.2) (layer "F.Cu") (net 8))
 (via (at 123.5725 78.9) (size 0.6) (drill 0.3) (layers "F.Cu" "B.Cu") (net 8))
 (via (at 115 107.4) (size 0.6) (drill 0.3) (layers "F.Cu" "B.Cu") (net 1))
 (segment (start 118.075 110.475) (end 115 107.4) (width 0.2) (layer "B.Cu") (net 1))
 (segment (start 130.825 110.475) (end 118.075 110.475) (width 0.2) (layer "B.Cu") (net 1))
 (via (at 115 104.6) (size 0.6) (drill 0.3) (layers "F.Cu" "B.Cu") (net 2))
 (segment (start 115.075 102) (end 115.075 104.525) (width 0.2) (layer "B.Cu") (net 2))
 (segment (start 115.075 104.525) (end 115 104.6) (width 0.2) (layer "B.Cu") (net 2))
 (via (at 129.5 96.9) (size 0.6) (drill 0.3) (layers "F.Cu" "B.Cu") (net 10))
 (segment (start 131.025 78.825) (end 131.025 95.375) (width 0.2) (layer "B.Cu") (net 10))
 (segment (start 131.025 95.375) (end 129.5 96.9) (width 0.2) (layer "B.Cu") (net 10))
 (via (at 129.5 94.1) (size 0.6) (drill 0.3) (layers "F.Cu" "B.Cu") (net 11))
 (segment (start 129.5 99.0375) (end 128.899 98.4365) (width 0.2) (layer "B.Cu") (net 11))
 (segment (start 128.899 94.701) (end 129.5 94.1) (width 0.2) (layer "B.Cu") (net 11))
 (segment (start 128.899 98.4365) (end 128.899 94.701) (width 0.2) (layer "B.Cu") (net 11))
 (segment (start 117.36805 102.269) (end 120.519 99.11805) (width 0.2) (layer "F.Cu") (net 6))
 (segment (start 112 105.96) (end 110.849 104.809) (width 0.2) (layer "F.Cu") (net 6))
 (segment (start 110.849 102.269) (end 117.36805 102.269) (width 0.2) (layer "F.Cu") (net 6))
 (segment (start 110.849 104.809) (end 110.849 102.269) (width 0.2) (layer "F.Cu") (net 6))
 (segment (start 120.519 99.11805) (end 120.519 97.561) (width 0.2) (layer "F.Cu") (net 6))
 (segment (start 120.519 97.561) (end 126.7 91.38) (width 0.2) (layer "F.Cu") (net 6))
 (segment (start 124.525 112.755) (end 118.795 112.755) (width 0.2) (layer "B.Cu") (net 6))
 (segment (start 118.795 112.755) (end 112 105.96) (width 0.2) (layer "B.Cu") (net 6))
 (segment (start 118.5 86.61384) (end 118.5 88.5) (width 0.2) (layer "F.Cu") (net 5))
 (segment (start 118 103.42) (end 112 103.42) (width 0.2) (layer "F.Cu") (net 5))
 (segment (start 129.5 101.8) (end 129.5 101.9625) (width 0.2) (layer "F.Cu") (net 5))
 (segment (start 122.28 103.42) (end 118 103.42) (width 0.2) (layer "F.Cu") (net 5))
 (segment (start 126.7 99) (end 129.5 101.8) (width 0.2) (layer "F.Cu") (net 5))
 (segment (start 116.86016 84.974) (end 118.5 86.61384) (width 0.2) (layer "F.Cu") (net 5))
 (segment (start 126.7 99) (end 122.28 103.42) (width 0.2) (layer "F.Cu") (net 5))
 (segment (start 112.5 81.96) (end 115.514 84.974) (width 0.2) (layer "F.Cu") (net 5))
 (segment (start 115.514 84.974) (end 116.86016 84.974) (width 0.2) (layer "F.Cu") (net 5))
 (via (at 118.5 88.5) (size 0.6) (drill 0.3) (layers "F.Cu" "B.Cu") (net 5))
 (via (at 129.5 101.9625) (size 0.6) (drill 0.3) (layers "F.Cu" "B.Cu") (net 5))
 (via (at 118 103.42) (size 0.6) (drill 0.3) (layers "F.Cu" "B.Cu") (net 5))
 (segment (start 115.101 99.45605) (end 115.101 95.021) (width 0.2) (layer "B.Cu") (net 5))
 (segment (start 117.9375 89.0625) (end 117.9375 92.1845) (width 0.2) (layer "B.Cu") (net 5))
 (segment (start 112 102.55705) (end 115.101 99.45605) (width 0.2) (layer "B.Cu") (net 5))
 (segment (start 112 103.42) (end 112 102.55705) (width 0.2) (layer "B.Cu") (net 5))
 (segment (start 132.5 98.9625) (end 129.5 101.9625) (width 0.2) (layer "B.Cu") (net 5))
 (segment (start 118 102) (end 118 103.42) (width 0.2) (layer "B.Cu") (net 5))
 (segment (start 115.101 95.021) (end 111.46 91.38) (width 0.2) (layer "B.Cu") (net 5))
 (segment (start 118.5 88.5) (end 117.9375 89.0625) (width 0.2) (layer "B.Cu") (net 5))
 (segment (start 117.9375 92.1845) (end 115.101 95.021) (width 0.2) (layer "B.Cu") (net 5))
 (segment (start 132.5 98) (end 132.5 98.9625) (width 0.2) (layer "B.Cu") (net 5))
 (segment (start 114 88.54) (end 114 91.38) (width 0.2) (layer "F.Cu") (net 4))
 (segment (start 121.62 85.62) (end 121.62 85.5275) (width 0.2) (layer "F.Cu") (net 4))
 (segment (start 121.74 85.5) (end 121.62 85.62) (width 0.2) (layer "F.Cu") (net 4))
 (segment (start 132.5 92.92) (end 128.745 89.165) (width 0.2) (layer "F.Cu") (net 4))
 (segment (start 128.745 89.165) (end 128.745 85.5) (width 0.2) (layer "F.Cu") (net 4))
 (segment (start 119.08 99) (end 119.08 91.38) (width 0.2) (layer "F.Cu") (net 4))
 (segment (start 121.62 91.38) (end 119.08 91.38) (width 0.2) (layer "F.Cu") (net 4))
 (segment (start 124.22 108.5) (end 124.525 108.195) (width 0.2) (layer "F.Cu") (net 4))
 (segment (start 121.62 85.5275) (end 121.2925 85.2) (width 0.2) (layer "F.Cu") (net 4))
 (segment (start 116.54 91.38) (end 119.08 91.38) (width 0.2) (layer "F.Cu") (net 4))
 (segment (start 116.54 99) (end 119.08 99) (width 0.2) (layer "F.Cu") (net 4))
 (segment (start 112.5 87.04) (end 114 88.54) (width 0.2) (layer "F.Cu") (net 4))
 (segment (start 114 99) (end 116.54 99) (width 0.2) (layer "F.Cu") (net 4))
 (segment (start 112 108.5) (end 124.22 108.5) (width 0.2) (layer "F.Cu") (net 4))
 (segment (start 128.745 85.5) (end 128.745 85.125) (width 0.2) (layer "F.Cu") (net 4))
 (segment (start 124.16 99) (end 121.62 99) (width 0.2) (layer "F.Cu") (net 4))
 (segment (start 116.54 91.38) (end 114 91.38) (width 0.2) (layer "F.Cu") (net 4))
 (via (at 121.2925 85.2) (size 0.6) (drill 0.3) (layers "F.Cu" "B.Cu") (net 4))
 (via (at 124.525 108.195) (size 0.6) (drill 0.3) (layers "F.Cu" "B.Cu") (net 4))
 (via (at 128.745 85.125) (size 0.6) (drill 0.3) (layers "F.Cu" "B.Cu") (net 4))
 (segment (start 121.2925 86.7925) (end 121.62 87.12) (width 0.2) (layer "B.Cu") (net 4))
 (segment (start 122.6935 86.601) (end 127.269 86.601) (width 0.2) (layer "B.Cu") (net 4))
 (segment (start 121.62 99) (end 119.08 99) (width 0.2) (layer "B.Cu") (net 4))
 (segment (start 112 108.5) (end 110.849 107.349) (width 0.2) (layer "B.Cu") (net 4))
 (segment (start 121.62 87.12) (end 121.62 91.38) (width 0.2) (layer "B.Cu") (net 4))
 (segment (start 110.849 102.151) (end 114 99) (width 0.2) (layer "B.Cu") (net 4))
 (segment (start 127.269 86.601) (end 128.745 85.125) (width 0.2) (layer "B.Cu") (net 4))
 (segment (start 121.2925 85.2) (end 122.6935 86.601) (width 0.2) (layer "B.Cu") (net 4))
 (segment (start 110.849 107.349) (end 110.849 102.151) (width 0.2) (layer "B.Cu") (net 4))
 (segment (start 121.2925 85.2) (end 121.2925 86.7925) (width 0.2) (layer "B.Cu") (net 4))
 (segment (start 112.561 97.899) (end 112.561 88.96) (width 0.2) (layer "F.Cu") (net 3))
 (segment (start 112.561 88.96) (end 111.349 87.748) (width 0.2) (layer "F.Cu") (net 3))
 (segment (start 111.46 99) (end 112.561 97.899) (width 0.2) (layer "F.Cu") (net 3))
 (segment (start 111.349 85.651) (end 112.5 84.5) (width 0.2) (layer "F.Cu") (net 3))
 (segment (start 111.349 87.748) (end 111.349 85.651) (width 0.2) (layer "F.Cu") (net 3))
 (segment (start 112.5 84.5) (end 113.35 83.65) (width 0.2) (layer "B.Cu") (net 3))
 (segment (start 113.35 83.65) (end 124.3025 83.65) (width 0.2) (layer "B.Cu") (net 3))
 (segment (start 124.3025 83.65) (end 125.8525 85.2) (width 0.2) (layer "B.Cu") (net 3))
 (segment (start 128.23124 90.279) (end 132.5 94.54776) (width 0.2) (layer "F.Cu") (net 7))
 (segment (start 132.5 94.54776) (end 132.5 95.46) (width 0.2) (layer "F.Cu") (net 7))
 (segment (start 124.16 91.38) (end 125.261 90.279) (width 0.2) (layer "F.Cu") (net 7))
 (segment (start 125.261 90.279) (end 128.23124 90.279) (width 0.2) (layer "F.Cu") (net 7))
 (segment (start 133.905 85.725) (end 133.905 94.055) (width 0.2) (layer "B.Cu") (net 7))
 (segment (start 133.305 85.125) (end 133.905 85.725) (width 0.2) (layer "B.Cu") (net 7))
 (segment (start 133.905 94.055) (end 132.5 95.46) (width 0.2) (layer "B.Cu") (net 7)))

